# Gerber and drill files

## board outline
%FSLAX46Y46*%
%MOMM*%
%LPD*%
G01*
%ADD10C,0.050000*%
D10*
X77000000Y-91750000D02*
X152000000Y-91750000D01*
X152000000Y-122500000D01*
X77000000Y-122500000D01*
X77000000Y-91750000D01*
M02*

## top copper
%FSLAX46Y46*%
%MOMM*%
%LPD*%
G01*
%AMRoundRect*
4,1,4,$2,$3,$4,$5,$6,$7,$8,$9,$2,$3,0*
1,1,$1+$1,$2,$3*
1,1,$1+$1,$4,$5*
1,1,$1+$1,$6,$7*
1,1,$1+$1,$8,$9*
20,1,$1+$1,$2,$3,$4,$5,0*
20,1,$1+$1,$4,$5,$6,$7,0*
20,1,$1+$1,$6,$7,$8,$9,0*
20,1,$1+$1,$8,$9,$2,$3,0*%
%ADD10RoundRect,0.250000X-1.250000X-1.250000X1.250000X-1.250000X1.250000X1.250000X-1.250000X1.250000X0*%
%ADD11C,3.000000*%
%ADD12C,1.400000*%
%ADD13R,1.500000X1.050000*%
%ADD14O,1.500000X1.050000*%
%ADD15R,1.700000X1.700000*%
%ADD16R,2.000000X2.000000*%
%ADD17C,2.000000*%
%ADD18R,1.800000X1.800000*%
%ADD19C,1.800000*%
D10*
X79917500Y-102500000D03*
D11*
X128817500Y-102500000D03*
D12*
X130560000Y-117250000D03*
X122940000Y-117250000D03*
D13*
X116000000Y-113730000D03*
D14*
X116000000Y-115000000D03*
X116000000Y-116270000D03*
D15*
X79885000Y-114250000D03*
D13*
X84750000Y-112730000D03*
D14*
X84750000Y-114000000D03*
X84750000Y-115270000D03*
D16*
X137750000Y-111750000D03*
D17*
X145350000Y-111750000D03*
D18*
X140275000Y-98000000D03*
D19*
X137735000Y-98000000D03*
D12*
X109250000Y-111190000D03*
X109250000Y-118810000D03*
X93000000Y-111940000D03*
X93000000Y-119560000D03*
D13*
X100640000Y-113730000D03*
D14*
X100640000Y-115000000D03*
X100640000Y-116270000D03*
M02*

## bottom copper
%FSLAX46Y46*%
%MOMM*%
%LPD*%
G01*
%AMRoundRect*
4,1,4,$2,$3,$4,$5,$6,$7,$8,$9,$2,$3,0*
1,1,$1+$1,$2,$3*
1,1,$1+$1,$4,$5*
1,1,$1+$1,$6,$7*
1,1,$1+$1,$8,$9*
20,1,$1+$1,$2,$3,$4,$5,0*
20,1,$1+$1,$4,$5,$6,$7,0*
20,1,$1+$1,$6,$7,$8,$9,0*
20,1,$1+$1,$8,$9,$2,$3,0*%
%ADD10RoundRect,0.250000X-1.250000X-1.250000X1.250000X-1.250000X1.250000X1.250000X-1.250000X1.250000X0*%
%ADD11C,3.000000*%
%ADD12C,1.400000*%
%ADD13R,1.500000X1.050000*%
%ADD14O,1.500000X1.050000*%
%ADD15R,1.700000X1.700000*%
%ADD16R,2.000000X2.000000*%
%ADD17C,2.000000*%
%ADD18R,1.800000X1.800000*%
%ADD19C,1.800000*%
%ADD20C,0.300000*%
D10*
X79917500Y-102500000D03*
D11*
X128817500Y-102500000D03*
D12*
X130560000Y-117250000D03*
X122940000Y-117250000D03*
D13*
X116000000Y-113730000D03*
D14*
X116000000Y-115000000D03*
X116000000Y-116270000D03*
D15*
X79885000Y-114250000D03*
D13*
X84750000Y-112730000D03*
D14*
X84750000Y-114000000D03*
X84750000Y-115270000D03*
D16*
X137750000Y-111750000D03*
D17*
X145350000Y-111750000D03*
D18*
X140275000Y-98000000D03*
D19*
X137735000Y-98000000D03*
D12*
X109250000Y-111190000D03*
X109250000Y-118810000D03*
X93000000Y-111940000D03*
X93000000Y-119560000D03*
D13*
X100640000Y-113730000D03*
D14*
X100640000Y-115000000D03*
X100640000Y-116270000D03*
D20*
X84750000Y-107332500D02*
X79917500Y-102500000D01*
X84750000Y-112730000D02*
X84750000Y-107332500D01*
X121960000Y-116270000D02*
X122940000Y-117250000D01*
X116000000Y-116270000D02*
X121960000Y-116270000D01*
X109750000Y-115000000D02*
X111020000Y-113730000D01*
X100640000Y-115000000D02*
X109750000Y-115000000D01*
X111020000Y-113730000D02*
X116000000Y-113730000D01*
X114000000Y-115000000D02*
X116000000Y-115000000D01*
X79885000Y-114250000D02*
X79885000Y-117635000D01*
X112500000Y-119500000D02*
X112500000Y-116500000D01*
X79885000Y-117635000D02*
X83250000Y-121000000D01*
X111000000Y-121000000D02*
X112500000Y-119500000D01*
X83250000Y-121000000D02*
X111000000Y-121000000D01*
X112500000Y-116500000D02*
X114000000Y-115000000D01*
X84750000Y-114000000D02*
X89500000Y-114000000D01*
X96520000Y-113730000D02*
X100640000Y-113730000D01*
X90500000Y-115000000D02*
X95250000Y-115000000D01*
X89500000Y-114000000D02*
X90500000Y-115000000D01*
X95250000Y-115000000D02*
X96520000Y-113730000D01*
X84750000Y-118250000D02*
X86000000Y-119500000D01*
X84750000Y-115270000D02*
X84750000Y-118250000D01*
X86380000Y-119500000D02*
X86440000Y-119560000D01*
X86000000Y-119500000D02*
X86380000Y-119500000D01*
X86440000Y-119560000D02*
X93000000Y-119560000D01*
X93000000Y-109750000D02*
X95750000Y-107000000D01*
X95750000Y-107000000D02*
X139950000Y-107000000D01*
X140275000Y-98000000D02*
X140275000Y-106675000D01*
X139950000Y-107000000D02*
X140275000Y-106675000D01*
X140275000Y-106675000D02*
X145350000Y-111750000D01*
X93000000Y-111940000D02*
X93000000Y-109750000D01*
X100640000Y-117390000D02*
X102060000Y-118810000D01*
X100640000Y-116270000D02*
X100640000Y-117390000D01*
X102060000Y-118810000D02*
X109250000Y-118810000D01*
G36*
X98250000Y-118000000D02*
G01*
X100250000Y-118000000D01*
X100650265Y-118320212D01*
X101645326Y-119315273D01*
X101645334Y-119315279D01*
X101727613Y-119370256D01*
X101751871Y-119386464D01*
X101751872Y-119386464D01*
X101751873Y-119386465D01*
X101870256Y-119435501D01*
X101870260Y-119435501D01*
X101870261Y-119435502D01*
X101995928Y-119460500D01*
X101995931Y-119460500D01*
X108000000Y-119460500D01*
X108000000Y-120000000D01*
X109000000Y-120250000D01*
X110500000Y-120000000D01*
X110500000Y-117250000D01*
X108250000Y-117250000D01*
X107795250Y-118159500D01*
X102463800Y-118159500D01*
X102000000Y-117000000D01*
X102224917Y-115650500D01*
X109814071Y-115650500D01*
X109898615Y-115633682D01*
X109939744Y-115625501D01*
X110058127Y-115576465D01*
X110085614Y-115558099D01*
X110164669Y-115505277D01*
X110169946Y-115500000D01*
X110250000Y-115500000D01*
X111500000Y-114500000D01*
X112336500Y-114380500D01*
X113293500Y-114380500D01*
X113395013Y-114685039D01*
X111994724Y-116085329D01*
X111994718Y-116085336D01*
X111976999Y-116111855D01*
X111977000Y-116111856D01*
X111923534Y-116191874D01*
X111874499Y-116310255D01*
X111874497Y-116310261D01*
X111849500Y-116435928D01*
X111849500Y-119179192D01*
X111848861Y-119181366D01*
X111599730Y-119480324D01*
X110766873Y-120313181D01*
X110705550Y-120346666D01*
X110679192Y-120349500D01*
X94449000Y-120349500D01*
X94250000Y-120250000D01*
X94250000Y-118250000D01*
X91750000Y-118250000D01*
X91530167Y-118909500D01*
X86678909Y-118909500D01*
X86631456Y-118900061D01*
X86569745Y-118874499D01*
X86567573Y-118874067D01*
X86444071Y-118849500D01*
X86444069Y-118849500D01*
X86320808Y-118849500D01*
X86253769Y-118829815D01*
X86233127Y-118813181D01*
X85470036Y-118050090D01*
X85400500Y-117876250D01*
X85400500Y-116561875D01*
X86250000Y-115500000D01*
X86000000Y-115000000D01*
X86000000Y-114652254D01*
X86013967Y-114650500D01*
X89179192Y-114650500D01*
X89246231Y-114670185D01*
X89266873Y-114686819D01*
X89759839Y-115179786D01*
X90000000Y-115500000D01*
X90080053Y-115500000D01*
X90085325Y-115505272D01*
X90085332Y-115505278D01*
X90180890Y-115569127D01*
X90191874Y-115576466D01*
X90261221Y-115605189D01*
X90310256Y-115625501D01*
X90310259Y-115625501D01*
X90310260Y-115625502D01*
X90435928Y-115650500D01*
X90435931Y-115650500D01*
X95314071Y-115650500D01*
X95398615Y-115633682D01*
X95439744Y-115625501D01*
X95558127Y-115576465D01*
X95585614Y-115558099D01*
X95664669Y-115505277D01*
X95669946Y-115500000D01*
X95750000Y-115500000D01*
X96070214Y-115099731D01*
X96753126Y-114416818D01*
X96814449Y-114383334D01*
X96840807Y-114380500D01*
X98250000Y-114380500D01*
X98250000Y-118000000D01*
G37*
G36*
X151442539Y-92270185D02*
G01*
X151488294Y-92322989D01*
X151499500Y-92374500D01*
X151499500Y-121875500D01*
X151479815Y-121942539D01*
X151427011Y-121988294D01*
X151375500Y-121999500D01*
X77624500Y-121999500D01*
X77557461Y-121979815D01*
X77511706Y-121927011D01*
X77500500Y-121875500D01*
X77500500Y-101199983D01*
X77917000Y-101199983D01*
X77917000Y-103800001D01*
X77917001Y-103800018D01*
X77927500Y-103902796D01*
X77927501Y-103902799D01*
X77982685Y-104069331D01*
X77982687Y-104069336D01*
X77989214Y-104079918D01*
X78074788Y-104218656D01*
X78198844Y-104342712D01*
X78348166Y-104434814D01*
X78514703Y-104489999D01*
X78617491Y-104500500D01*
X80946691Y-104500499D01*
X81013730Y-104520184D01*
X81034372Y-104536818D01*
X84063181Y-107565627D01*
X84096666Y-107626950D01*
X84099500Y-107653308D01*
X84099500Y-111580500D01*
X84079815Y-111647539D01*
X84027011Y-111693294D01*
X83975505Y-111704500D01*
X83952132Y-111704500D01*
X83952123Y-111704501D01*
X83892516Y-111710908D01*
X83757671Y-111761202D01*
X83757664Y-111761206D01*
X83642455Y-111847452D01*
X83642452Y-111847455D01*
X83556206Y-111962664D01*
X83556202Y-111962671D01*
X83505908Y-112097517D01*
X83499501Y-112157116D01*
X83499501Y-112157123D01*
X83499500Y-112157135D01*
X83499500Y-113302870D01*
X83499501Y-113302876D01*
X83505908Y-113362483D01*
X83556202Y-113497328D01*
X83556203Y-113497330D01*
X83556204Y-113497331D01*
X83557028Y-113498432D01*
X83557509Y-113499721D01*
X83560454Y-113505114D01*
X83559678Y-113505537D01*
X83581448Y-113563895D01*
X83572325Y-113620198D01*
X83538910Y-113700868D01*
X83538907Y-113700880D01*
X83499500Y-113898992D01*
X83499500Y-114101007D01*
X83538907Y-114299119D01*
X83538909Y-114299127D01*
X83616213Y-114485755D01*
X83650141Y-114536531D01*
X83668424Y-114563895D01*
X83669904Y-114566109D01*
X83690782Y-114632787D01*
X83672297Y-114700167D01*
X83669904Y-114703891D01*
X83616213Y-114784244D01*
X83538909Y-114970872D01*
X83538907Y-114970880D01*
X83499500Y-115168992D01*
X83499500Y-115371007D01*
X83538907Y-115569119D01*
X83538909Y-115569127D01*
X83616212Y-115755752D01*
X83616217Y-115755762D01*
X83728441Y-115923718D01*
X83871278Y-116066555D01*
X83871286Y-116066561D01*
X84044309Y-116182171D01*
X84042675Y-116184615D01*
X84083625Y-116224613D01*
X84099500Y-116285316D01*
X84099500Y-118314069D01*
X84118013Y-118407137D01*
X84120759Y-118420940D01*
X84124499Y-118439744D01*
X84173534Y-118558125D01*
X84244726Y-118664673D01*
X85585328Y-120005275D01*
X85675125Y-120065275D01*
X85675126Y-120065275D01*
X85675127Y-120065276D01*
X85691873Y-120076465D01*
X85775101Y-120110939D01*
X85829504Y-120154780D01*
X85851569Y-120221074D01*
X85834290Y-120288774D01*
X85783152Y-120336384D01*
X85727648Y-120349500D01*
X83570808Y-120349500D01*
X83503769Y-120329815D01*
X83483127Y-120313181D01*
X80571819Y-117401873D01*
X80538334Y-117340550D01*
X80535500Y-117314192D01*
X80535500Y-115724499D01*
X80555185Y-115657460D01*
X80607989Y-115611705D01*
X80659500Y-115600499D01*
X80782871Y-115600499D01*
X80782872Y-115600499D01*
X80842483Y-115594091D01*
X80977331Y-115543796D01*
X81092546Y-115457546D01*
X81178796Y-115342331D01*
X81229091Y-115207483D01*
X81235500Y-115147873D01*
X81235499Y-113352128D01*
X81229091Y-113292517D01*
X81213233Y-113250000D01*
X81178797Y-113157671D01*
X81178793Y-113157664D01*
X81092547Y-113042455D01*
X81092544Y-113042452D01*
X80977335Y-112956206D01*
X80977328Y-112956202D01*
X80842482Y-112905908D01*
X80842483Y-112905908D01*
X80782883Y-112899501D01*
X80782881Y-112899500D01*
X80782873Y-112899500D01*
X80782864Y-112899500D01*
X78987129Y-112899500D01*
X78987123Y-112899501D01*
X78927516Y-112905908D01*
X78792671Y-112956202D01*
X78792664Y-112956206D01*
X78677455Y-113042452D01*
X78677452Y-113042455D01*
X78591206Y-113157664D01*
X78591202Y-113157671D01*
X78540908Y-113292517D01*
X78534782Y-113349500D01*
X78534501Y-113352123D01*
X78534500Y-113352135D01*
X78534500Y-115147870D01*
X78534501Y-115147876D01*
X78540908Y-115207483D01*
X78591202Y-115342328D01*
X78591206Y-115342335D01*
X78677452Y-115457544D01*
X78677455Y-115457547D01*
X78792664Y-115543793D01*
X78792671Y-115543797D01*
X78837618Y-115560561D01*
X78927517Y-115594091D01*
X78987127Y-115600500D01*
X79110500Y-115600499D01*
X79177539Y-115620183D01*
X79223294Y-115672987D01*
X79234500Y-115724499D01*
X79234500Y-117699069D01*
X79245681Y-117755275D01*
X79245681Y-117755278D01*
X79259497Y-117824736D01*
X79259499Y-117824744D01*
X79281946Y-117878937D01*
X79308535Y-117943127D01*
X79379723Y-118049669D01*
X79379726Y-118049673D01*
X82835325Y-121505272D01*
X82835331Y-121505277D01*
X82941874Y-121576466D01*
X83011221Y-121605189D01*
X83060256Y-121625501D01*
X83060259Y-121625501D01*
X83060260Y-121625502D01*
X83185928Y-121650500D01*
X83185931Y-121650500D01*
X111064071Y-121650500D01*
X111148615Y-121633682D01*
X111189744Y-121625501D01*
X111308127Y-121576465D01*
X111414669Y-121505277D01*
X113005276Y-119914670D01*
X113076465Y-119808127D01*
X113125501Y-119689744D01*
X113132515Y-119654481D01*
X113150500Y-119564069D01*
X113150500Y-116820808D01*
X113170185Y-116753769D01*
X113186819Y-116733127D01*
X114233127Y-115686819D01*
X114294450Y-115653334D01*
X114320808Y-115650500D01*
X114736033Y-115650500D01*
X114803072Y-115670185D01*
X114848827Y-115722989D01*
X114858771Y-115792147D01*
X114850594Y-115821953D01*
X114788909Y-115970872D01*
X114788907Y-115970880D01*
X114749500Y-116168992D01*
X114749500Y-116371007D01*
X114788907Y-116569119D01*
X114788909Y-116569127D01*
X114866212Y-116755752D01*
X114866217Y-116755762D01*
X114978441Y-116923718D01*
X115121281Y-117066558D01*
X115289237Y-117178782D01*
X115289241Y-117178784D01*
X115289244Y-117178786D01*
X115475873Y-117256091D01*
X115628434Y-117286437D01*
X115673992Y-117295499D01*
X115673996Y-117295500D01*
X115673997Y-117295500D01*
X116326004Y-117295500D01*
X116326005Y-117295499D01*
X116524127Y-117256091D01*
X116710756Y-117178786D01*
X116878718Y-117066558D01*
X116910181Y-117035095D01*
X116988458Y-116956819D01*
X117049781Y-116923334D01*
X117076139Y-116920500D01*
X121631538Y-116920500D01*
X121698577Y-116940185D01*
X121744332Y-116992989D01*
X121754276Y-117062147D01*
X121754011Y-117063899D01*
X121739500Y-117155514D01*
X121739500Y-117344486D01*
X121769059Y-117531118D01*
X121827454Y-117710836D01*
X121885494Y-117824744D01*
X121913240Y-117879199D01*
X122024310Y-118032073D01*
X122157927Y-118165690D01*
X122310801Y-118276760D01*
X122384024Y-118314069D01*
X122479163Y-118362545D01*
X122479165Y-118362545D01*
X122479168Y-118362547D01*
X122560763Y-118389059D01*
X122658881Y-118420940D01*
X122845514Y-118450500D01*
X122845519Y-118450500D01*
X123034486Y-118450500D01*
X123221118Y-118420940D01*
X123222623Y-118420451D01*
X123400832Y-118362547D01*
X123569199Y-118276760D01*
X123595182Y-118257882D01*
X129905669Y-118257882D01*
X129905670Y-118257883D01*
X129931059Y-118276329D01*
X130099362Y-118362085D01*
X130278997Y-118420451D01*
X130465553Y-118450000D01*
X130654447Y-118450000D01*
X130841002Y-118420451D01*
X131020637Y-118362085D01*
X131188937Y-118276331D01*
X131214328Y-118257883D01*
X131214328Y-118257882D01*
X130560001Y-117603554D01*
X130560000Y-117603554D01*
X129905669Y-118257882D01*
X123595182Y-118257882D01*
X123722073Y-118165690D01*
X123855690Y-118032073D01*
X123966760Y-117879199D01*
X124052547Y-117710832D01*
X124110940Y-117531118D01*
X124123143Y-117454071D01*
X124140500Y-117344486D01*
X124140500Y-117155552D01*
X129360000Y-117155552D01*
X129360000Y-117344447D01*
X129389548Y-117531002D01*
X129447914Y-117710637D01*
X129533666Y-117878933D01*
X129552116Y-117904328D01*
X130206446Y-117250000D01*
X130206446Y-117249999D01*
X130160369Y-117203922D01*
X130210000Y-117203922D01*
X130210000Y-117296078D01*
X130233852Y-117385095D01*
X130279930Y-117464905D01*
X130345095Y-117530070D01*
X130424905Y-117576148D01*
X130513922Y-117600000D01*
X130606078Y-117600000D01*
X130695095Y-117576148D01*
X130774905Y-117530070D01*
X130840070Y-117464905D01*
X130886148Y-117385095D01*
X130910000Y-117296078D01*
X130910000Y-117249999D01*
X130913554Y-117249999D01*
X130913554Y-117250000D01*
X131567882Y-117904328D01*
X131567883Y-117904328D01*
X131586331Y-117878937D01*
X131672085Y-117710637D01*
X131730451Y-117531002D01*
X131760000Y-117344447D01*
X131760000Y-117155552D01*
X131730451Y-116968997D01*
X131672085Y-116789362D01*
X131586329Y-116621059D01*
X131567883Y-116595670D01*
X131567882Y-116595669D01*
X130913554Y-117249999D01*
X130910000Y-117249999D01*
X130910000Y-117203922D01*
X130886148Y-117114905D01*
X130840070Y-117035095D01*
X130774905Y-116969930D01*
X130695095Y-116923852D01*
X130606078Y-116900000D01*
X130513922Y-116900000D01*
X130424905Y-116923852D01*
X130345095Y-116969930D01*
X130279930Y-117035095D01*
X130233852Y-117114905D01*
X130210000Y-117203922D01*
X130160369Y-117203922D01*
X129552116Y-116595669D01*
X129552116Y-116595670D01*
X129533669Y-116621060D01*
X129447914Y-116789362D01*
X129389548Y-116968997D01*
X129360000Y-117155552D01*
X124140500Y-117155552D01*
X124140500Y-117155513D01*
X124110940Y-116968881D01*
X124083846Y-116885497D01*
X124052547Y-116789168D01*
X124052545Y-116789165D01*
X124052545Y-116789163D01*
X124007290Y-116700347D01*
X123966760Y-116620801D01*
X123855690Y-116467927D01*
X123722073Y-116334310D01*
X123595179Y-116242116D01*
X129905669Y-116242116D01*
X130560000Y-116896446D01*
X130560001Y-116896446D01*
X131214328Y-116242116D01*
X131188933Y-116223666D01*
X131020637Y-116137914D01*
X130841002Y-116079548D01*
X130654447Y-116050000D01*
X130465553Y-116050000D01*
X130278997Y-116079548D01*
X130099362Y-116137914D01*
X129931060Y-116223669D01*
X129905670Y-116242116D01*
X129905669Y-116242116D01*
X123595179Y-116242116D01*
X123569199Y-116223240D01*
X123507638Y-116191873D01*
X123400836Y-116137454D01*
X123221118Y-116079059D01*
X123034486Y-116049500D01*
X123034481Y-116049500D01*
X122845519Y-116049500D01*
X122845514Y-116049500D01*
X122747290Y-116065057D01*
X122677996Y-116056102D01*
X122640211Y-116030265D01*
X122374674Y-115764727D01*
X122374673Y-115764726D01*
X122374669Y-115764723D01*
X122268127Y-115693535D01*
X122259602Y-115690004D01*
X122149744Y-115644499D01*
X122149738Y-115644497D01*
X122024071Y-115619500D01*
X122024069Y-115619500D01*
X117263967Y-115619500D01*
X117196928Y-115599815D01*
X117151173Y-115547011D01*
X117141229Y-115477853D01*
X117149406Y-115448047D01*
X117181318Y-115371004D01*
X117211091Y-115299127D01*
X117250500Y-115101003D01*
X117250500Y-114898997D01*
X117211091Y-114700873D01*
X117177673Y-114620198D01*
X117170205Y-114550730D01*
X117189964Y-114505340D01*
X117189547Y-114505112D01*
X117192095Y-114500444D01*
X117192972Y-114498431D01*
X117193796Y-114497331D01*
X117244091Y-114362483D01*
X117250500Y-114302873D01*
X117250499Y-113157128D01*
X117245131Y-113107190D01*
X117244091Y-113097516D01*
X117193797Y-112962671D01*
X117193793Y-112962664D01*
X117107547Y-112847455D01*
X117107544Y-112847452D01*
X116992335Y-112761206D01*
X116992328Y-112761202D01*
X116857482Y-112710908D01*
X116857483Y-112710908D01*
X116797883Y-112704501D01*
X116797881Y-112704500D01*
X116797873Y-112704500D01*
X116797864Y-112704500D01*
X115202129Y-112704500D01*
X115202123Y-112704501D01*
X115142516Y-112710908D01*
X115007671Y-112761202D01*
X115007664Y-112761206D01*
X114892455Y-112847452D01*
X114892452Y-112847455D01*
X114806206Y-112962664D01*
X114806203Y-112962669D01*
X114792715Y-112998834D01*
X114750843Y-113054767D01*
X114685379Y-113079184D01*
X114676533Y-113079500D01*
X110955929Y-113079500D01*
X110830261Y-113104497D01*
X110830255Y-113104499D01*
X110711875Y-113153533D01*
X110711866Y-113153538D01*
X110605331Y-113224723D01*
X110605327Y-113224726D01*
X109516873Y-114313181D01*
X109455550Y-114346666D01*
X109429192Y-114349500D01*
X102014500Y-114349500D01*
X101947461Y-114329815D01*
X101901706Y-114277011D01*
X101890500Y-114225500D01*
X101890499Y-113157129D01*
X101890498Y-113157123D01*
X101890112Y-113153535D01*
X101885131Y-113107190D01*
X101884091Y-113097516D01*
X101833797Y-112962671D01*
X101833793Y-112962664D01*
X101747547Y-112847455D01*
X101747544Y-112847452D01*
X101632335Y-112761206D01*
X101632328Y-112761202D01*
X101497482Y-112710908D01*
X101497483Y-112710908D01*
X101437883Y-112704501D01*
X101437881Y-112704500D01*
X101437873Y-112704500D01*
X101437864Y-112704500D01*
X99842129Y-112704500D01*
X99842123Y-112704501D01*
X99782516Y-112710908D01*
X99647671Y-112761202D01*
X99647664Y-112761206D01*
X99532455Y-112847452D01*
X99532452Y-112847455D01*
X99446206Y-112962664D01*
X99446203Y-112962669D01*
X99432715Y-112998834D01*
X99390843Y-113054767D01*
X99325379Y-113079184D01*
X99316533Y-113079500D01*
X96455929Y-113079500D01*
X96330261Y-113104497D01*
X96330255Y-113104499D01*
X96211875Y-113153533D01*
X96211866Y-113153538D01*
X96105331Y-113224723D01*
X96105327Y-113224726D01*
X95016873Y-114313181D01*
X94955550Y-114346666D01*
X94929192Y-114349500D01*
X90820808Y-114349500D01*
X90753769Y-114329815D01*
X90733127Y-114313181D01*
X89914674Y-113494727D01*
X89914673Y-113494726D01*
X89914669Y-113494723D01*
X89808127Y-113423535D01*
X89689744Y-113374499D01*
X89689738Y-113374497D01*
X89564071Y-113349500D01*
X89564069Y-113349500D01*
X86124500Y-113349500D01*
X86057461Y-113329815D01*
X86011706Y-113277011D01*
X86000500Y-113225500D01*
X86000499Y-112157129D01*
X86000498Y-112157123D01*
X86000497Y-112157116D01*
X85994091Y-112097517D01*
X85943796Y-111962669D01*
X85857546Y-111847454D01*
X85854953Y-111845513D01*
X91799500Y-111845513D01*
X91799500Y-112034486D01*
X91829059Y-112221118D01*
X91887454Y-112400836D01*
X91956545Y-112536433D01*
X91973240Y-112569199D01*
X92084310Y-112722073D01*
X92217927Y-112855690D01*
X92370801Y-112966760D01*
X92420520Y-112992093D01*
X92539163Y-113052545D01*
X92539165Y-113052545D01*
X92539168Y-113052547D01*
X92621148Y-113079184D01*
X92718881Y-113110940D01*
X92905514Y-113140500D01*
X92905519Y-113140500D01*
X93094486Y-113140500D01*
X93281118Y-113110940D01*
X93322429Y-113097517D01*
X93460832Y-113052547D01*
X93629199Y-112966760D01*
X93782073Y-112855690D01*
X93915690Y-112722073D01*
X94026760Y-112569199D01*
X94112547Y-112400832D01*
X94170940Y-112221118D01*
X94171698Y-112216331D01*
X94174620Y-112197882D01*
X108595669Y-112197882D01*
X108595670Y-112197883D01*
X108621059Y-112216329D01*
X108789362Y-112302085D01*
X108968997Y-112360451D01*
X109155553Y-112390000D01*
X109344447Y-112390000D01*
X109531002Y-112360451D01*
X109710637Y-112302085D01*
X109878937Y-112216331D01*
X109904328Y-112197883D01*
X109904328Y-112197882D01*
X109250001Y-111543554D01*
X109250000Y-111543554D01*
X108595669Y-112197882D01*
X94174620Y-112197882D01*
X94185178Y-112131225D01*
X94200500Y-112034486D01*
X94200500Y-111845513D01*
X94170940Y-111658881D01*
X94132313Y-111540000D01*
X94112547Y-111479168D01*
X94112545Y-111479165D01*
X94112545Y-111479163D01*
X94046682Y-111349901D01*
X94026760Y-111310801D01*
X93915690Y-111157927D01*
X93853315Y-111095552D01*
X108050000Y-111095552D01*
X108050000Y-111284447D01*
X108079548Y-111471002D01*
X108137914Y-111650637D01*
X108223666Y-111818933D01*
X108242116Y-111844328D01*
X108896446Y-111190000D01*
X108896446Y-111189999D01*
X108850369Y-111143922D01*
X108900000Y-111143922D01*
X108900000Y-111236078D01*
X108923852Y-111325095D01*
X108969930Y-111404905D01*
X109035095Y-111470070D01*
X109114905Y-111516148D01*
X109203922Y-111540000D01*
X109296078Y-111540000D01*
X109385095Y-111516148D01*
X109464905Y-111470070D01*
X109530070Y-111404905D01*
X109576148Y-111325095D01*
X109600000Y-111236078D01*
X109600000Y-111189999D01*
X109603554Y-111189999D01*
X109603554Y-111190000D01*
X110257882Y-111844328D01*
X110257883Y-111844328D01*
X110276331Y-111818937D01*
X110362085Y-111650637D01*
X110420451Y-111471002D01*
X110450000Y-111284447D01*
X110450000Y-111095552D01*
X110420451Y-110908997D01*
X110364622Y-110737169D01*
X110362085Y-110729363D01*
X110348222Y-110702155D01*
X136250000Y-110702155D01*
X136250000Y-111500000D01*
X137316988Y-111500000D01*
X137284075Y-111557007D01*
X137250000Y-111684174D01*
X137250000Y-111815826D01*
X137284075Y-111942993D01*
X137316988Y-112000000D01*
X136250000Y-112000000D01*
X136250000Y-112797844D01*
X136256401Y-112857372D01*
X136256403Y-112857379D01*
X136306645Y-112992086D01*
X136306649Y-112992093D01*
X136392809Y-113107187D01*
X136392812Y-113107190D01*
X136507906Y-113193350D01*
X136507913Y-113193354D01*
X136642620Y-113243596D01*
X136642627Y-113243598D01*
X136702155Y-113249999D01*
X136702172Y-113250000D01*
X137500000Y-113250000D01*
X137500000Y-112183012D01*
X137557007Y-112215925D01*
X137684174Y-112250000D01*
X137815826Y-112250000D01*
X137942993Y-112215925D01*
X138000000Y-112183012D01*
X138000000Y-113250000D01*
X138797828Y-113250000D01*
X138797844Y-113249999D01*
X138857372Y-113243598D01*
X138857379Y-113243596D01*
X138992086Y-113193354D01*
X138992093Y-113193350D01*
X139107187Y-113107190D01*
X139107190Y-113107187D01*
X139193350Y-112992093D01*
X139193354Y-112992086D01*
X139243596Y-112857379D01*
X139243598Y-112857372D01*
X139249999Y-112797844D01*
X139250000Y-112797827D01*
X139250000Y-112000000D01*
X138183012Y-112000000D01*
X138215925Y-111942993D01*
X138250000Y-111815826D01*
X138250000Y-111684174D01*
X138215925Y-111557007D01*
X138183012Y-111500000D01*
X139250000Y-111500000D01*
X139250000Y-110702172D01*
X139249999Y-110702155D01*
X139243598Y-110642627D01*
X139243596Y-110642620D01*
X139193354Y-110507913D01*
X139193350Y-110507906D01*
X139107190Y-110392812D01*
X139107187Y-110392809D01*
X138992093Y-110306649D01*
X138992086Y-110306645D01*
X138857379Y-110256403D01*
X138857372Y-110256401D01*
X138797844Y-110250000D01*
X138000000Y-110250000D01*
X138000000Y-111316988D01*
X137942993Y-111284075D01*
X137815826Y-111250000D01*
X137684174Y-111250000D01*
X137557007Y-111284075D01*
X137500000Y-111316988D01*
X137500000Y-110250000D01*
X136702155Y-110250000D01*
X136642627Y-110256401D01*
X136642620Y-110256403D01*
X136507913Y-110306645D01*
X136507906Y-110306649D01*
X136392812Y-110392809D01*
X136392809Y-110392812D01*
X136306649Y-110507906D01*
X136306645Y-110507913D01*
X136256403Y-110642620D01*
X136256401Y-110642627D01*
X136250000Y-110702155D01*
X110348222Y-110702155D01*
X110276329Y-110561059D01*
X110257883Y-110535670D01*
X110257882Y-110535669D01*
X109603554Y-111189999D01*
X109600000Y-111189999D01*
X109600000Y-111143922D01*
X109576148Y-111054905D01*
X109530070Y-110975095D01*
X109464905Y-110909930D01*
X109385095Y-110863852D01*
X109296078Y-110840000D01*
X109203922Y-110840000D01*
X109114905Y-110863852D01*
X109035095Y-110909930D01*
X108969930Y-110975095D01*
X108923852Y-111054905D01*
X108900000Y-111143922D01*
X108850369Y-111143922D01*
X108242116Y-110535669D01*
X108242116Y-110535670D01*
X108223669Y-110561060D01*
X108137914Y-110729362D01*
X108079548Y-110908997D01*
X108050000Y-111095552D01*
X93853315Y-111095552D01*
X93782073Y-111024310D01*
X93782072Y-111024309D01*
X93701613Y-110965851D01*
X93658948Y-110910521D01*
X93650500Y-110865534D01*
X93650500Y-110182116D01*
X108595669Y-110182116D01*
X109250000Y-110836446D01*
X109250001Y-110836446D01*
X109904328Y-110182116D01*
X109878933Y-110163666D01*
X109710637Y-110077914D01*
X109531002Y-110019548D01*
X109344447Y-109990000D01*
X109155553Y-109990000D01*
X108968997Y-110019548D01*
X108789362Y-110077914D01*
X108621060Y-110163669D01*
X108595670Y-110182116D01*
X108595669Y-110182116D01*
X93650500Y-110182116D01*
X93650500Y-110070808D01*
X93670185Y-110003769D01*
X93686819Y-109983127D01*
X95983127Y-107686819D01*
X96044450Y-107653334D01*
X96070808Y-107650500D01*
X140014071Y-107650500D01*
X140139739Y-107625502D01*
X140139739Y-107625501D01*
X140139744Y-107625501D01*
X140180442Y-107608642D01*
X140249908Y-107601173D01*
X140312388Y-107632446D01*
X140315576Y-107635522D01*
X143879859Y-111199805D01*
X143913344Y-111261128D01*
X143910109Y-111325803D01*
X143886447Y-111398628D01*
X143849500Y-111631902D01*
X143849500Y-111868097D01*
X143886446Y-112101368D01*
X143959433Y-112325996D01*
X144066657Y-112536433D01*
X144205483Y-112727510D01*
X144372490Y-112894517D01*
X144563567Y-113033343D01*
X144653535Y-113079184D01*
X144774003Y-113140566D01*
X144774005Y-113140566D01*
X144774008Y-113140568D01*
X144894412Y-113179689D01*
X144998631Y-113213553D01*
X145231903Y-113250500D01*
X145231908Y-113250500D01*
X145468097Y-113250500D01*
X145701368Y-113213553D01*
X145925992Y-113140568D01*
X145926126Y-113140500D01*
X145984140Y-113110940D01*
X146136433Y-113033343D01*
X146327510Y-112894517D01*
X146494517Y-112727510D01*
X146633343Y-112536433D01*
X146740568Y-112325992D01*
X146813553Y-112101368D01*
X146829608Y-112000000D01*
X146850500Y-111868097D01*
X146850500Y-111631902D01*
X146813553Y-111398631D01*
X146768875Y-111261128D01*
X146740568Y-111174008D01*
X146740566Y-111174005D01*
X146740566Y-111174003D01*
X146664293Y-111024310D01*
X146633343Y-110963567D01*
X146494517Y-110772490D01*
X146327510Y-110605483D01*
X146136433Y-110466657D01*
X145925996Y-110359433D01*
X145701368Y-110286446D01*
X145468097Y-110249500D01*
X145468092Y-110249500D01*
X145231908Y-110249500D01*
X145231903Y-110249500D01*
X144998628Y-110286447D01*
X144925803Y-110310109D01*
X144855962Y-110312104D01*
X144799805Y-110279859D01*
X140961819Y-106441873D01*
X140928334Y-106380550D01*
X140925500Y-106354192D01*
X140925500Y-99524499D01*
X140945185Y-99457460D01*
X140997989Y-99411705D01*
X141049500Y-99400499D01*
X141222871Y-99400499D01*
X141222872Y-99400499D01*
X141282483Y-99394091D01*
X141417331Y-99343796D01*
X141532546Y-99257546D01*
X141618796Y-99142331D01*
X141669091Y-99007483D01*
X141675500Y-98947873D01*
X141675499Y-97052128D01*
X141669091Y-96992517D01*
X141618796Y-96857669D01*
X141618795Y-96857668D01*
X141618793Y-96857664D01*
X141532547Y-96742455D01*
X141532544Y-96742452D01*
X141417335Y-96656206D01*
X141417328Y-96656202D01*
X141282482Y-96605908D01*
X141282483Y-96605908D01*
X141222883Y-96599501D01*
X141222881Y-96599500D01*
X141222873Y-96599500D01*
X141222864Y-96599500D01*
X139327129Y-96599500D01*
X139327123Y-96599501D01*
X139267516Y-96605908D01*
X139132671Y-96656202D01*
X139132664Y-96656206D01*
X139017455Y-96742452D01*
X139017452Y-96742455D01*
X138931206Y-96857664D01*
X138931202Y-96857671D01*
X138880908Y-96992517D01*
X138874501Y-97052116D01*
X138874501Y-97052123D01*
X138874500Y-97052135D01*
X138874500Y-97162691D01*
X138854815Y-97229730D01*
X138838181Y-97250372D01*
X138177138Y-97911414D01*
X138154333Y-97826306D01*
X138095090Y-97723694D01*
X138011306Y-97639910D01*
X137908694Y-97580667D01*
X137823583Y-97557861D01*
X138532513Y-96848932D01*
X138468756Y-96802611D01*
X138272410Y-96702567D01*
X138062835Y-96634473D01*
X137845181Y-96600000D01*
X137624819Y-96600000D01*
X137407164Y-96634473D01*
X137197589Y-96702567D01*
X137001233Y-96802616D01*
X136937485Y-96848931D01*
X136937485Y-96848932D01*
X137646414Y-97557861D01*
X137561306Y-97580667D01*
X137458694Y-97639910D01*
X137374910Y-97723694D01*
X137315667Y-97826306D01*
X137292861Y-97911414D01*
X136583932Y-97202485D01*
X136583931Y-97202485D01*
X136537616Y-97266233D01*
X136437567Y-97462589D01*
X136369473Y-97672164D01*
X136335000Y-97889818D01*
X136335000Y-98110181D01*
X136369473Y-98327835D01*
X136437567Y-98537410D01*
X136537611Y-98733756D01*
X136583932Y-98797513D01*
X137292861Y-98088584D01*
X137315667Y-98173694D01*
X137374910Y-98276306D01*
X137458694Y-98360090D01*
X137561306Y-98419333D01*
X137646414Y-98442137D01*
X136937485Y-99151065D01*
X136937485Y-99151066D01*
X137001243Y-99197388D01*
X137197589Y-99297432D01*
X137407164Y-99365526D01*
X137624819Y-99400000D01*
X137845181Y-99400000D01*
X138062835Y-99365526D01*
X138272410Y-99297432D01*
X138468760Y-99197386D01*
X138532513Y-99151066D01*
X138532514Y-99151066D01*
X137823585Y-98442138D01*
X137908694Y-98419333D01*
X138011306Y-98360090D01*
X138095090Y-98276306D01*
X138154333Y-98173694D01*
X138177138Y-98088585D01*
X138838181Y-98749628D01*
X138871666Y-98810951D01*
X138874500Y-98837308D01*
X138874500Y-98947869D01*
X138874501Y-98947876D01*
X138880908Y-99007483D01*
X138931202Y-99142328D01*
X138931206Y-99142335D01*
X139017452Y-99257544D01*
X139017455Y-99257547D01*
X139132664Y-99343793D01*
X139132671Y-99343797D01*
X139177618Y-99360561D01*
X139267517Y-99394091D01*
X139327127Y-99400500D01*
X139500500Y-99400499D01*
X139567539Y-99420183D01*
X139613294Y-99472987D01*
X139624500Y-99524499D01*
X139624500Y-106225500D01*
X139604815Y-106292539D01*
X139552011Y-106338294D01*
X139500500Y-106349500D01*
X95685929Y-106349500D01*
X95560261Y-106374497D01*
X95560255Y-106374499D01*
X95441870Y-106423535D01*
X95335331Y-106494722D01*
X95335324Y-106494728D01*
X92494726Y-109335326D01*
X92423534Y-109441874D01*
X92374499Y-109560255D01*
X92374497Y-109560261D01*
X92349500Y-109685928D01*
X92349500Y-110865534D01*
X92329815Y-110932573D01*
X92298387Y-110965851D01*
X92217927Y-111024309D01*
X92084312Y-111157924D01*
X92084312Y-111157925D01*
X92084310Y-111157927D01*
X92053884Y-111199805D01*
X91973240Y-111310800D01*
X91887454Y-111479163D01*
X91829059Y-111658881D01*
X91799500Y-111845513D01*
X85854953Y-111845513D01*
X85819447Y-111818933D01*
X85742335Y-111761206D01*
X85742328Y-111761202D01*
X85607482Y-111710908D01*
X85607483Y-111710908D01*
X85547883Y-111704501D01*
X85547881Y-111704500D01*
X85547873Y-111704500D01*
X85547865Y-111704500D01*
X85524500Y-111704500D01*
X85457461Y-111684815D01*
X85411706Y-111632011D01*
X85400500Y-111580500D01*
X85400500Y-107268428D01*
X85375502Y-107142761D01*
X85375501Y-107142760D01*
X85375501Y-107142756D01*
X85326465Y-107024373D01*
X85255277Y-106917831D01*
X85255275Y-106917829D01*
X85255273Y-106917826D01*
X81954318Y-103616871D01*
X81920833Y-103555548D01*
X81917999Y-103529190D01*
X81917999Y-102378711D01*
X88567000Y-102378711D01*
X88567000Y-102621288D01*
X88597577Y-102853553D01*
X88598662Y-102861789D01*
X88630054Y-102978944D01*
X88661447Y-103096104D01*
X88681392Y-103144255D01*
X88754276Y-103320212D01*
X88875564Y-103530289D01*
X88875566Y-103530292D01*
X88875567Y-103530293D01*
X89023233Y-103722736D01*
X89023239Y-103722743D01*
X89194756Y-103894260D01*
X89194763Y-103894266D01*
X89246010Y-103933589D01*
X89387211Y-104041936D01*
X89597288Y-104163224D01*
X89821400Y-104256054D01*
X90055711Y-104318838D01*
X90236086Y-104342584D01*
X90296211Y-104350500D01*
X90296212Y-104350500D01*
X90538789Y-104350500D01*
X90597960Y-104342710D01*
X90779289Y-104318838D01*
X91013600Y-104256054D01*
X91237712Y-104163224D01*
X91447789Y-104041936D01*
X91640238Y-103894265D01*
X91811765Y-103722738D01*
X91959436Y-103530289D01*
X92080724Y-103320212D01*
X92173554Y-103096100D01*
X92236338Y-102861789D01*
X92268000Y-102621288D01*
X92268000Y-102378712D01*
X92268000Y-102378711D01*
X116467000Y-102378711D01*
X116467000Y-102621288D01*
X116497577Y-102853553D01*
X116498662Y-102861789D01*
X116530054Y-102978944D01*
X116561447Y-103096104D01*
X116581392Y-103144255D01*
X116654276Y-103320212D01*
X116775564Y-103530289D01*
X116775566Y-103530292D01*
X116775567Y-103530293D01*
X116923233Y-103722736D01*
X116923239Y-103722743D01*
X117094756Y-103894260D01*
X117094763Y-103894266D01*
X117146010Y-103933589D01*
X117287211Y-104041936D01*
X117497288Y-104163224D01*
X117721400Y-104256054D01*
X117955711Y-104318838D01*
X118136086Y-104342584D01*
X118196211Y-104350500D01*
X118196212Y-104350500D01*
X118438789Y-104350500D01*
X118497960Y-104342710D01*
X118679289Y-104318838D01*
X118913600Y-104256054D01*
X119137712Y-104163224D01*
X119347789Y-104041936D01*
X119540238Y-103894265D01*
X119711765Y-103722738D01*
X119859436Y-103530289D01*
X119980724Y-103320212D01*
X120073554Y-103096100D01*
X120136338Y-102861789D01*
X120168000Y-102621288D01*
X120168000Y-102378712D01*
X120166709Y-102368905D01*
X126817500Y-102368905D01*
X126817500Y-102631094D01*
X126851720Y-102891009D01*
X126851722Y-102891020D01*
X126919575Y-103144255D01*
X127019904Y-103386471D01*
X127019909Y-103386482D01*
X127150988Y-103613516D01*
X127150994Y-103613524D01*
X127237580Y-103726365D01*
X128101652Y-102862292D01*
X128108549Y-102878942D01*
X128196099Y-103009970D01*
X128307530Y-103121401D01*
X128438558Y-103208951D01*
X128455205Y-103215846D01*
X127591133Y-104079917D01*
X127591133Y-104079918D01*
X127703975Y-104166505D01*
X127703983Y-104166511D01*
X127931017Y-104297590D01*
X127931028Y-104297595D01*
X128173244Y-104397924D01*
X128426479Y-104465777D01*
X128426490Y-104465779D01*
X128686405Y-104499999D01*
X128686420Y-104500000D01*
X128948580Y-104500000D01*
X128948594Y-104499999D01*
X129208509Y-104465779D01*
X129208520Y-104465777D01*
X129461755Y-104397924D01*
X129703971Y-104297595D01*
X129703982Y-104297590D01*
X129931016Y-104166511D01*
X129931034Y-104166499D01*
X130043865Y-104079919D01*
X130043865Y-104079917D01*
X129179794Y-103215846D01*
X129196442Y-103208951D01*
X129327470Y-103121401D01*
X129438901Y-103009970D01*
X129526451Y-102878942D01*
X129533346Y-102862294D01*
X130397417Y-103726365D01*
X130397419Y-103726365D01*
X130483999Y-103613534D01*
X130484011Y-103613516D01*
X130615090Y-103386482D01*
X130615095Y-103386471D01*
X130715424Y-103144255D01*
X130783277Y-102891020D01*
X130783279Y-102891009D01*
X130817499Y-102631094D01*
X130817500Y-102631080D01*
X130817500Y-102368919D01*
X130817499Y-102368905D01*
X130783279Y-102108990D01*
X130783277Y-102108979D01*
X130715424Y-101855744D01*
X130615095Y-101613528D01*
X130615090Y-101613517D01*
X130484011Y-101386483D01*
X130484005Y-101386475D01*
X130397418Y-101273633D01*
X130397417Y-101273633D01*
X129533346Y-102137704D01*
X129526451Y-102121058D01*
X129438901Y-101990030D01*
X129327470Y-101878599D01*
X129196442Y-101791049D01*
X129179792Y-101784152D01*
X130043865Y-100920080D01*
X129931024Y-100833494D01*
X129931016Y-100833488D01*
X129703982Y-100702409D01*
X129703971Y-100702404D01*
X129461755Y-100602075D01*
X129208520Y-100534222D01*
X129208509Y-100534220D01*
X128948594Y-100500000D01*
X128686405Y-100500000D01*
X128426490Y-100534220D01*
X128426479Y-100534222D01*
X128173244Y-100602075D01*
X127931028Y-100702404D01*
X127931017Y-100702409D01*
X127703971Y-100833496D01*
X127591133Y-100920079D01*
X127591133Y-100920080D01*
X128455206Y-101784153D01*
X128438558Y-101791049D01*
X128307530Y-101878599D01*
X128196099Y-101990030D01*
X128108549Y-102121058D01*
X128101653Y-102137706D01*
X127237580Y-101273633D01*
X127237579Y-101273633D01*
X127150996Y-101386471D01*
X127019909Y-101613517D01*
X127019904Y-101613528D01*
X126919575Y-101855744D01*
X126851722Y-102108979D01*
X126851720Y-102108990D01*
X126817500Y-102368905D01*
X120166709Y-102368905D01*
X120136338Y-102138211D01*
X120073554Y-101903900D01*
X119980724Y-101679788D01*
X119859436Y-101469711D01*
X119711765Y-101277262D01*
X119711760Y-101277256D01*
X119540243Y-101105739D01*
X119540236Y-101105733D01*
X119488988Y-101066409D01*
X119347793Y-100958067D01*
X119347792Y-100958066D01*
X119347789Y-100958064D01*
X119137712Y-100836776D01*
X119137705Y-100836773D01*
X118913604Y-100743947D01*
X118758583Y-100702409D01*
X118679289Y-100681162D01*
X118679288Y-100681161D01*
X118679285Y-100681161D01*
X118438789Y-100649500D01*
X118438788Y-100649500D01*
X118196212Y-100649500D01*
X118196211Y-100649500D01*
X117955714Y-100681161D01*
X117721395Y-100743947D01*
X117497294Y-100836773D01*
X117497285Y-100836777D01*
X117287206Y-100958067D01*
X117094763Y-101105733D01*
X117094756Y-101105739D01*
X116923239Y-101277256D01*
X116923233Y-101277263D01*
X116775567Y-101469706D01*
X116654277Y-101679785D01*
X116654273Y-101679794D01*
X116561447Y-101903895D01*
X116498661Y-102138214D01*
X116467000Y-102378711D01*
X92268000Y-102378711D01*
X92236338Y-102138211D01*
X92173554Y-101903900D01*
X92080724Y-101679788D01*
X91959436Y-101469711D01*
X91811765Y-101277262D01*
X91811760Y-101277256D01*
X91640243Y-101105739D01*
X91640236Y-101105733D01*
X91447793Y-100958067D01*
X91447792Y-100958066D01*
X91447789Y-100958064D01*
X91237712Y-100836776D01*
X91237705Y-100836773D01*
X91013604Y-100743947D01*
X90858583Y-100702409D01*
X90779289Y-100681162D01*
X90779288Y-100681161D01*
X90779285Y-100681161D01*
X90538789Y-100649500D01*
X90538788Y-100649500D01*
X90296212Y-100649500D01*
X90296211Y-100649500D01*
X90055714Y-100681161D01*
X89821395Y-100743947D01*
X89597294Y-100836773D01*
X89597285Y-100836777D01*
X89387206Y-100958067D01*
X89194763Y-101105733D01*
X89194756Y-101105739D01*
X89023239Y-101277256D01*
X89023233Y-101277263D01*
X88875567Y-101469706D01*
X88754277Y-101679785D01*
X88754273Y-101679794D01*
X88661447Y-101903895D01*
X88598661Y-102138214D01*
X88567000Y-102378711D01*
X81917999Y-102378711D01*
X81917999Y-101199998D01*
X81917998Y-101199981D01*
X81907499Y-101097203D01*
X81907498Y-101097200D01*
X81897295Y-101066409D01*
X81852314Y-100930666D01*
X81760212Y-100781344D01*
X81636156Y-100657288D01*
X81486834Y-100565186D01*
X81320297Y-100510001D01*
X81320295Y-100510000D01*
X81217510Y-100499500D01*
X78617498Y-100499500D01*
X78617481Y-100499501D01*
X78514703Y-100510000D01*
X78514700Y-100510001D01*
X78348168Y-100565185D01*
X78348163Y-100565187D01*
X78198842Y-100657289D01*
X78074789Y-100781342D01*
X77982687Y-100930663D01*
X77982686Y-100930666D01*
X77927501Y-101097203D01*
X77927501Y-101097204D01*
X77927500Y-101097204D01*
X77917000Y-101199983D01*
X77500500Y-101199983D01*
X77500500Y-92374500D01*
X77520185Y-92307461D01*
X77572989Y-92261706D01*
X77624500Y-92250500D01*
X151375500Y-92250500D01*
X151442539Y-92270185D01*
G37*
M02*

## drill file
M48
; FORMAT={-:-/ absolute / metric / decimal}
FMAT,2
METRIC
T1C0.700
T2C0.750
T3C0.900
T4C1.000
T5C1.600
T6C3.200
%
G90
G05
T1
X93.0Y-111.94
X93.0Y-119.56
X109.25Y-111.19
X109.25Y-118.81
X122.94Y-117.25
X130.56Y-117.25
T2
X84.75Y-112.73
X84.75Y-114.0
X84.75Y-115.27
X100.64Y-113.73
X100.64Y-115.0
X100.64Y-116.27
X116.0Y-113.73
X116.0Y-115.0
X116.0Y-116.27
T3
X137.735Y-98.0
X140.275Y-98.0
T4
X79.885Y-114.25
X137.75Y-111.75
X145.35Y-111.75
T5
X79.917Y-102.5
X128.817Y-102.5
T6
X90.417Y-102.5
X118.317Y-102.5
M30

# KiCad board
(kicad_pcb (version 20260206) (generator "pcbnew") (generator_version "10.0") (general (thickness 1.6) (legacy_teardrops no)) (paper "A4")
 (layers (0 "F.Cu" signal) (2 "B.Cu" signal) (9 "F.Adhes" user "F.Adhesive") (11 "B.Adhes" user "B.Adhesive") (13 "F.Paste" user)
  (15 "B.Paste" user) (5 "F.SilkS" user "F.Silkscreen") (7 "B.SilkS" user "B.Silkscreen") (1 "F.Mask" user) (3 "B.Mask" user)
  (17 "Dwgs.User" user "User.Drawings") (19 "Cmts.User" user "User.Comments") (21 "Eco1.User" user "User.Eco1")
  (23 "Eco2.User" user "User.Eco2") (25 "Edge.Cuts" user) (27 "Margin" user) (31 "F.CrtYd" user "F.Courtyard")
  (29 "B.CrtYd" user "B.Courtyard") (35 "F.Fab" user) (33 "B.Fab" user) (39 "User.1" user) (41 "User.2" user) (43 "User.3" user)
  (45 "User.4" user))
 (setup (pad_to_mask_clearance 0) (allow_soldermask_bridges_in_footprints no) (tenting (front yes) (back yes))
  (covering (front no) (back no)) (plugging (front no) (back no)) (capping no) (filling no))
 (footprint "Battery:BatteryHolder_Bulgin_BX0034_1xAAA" (layer "F.Cu") (at 79.9175 102.5)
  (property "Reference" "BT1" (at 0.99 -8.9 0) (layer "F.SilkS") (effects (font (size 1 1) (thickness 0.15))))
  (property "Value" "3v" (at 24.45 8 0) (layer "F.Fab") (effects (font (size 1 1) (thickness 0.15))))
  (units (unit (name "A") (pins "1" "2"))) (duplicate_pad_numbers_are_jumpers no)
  (pad "" np_thru_hole circle (at 10.5 0) (size 3.2 3.2) (drill 3.2) (layers "*.Cu" "*.Mask"))
  (pad "" np_thru_hole circle (at 38.4 0) (size 3.2 3.2) (drill 3.2) (layers "*.Cu" "*.Mask"))
  (pad "1" thru_hole roundrect (at 0 0) (size 3 3) (drill 1.6) (layers "*.Cu" "*.Mask") (remove_unused_layers no)
   (roundrect_rratio 0.08333333333) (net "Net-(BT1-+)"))
  (pad "2" thru_hole circle (at 48.9 0) (size 3 3) (drill 1.6) (layers "*.Cu" "*.Mask") (remove_unused_layers no) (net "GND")))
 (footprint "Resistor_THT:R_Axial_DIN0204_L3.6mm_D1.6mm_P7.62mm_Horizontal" (layer "F.Cu") (at 130.56 117.25 180)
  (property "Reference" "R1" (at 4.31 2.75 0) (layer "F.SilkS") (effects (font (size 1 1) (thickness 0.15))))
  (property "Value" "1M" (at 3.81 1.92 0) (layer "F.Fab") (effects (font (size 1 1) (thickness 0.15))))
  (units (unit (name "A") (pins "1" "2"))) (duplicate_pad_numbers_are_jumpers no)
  (pad "1" thru_hole circle (at 0 0 180) (size 1.4 1.4) (drill 0.7) (layers "*.Cu" "*.Mask") (remove_unused_layers no) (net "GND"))
  (pad "2" thru_hole circle (at 7.62 0 180) (size 1.4 1.4) (drill 0.7) (layers "*.Cu" "*.Mask") (remove_unused_layers no) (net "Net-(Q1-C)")))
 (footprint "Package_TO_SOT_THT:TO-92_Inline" (layer "F.Cu") (at 116 113.73 -90)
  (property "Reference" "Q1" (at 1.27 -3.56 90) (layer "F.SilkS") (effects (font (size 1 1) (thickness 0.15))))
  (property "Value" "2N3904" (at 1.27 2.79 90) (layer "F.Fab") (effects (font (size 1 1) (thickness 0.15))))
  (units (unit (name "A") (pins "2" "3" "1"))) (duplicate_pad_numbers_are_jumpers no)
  (pad "1" thru_hole rect (at 0 0 270) (size 1.05 1.5) (drill 0.75) (layers "*.Cu" "*.Mask") (remove_unused_layers no) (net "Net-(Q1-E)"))
  (pad "2" thru_hole oval (at 1.27 0 270) (size 1.05 1.5) (drill 0.75) (layers "*.Cu" "*.Mask") (remove_unused_layers no)
   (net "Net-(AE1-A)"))
  (pad "3" thru_hole oval (at 2.54 0 270) (size 1.05 1.5) (drill 0.75) (layers "*.Cu" "*.Mask") (remove_unused_layers no) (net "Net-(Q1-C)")))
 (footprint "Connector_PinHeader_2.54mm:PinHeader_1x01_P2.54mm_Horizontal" (layer "F.Cu") (at 79.885 114.25 180)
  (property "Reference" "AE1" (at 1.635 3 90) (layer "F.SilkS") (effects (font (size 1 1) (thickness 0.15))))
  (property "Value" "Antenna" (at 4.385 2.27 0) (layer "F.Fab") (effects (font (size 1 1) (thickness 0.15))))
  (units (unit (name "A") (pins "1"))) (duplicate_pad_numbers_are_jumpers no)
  (pad "1" thru_hole rect (at 0 0 180) (size 1.7 1.7) (drill 1) (layers "*.Cu" "*.Mask") (remove_unused_layers no) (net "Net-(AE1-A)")))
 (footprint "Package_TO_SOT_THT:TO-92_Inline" (layer "F.Cu") (at 84.75 112.73 -90)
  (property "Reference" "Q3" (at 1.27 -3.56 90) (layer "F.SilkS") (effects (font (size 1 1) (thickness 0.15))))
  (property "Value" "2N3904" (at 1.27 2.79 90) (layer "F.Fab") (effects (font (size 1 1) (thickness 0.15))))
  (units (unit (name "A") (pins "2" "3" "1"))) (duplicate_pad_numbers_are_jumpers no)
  (pad "1" thru_hole rect (at 0 0 270) (size 1.05 1.5) (drill 0.75) (layers "*.Cu" "*.Mask") (remove_unused_layers no) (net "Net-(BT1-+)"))
  (pad "2" thru_hole oval (at 1.27 0 270) (size 1.05 1.5) (drill 0.75) (layers "*.Cu" "*.Mask") (remove_unused_layers no) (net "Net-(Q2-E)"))
  (pad "3" thru_hole oval (at 2.54 0 270) (size 1.05 1.5) (drill 0.75) (layers "*.Cu" "*.Mask") (remove_unused_layers no) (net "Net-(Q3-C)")))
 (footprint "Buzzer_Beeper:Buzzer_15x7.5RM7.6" (layer "F.Cu") (at 137.75 111.75)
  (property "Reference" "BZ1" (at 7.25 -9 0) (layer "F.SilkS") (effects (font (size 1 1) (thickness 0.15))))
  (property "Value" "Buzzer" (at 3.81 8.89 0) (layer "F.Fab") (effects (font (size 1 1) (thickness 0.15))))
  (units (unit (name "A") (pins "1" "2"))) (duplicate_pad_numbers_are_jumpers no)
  (pad "1" thru_hole rect (at 0 0) (size 2 2) (drill 1) (layers "*.Cu" "*.Mask") (remove_unused_layers no) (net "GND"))
  (pad "2" thru_hole circle (at 7.6 0) (size 2 2) (drill 1) (layers "*.Cu" "*.Mask") (remove_unused_layers no) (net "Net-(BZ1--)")))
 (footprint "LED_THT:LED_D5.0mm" (layer "F.Cu") (at 140.275 98 180)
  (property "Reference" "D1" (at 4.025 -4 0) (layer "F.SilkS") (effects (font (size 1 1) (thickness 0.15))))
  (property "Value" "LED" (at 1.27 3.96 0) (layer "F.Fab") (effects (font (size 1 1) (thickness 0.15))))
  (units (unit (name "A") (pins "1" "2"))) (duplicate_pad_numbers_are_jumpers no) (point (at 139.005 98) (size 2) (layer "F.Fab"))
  (pad "1" thru_hole rect (at 0 0 180) (size 1.8 1.8) (drill 0.9) (layers "*.Cu" "*.Mask") (remove_unused_layers no) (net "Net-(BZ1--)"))
  (pad "2" thru_hole circle (at 2.54 0 180) (size 1.8 1.8) (drill 0.9) (layers "*.Cu" "*.Mask") (remove_unused_layers no) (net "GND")))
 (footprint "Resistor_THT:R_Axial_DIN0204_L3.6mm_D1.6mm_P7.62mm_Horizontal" (layer "F.Cu") (at 109.25 111.19 -90)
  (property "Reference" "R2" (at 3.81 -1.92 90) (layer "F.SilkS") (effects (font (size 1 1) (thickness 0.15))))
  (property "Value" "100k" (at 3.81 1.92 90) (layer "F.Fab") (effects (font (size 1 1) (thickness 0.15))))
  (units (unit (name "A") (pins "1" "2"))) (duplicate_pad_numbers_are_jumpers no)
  (pad "1" thru_hole circle (at 0 0 270) (size 1.4 1.4) (drill 0.7) (layers "*.Cu" "*.Mask") (remove_unused_layers no) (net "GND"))
  (pad "2" thru_hole circle (at 7.62 0 270) (size 1.4 1.4) (drill 0.7) (layers "*.Cu" "*.Mask") (remove_unused_layers no) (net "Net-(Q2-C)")))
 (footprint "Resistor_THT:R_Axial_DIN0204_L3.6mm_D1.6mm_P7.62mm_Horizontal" (layer "F.Cu") (at 93 111.94 -90)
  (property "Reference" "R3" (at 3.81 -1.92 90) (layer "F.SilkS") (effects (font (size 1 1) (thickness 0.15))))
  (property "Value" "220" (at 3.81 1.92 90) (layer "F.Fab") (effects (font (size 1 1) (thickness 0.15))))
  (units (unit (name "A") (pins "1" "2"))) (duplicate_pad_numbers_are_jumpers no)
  (pad "1" thru_hole circle (at 0 0 270) (size 1.4 1.4) (drill 0.7) (layers "*.Cu" "*.Mask") (remove_unused_layers no) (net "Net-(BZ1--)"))
  (pad "2" thru_hole circle (at 7.62 0 270) (size 1.4 1.4) (drill 0.7) (layers "*.Cu" "*.Mask") (remove_unused_layers no) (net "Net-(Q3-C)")))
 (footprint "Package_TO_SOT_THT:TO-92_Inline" (layer "F.Cu") (at 100.64 113.73 -90)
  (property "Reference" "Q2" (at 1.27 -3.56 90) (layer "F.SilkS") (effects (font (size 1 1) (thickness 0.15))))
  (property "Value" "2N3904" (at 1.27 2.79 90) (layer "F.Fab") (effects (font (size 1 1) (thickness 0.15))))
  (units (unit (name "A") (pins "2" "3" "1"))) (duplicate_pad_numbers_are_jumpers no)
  (pad "1" thru_hole rect (at 0 0 270) (size 1.05 1.5) (drill 0.75) (layers "*.Cu" "*.Mask") (remove_unused_layers no) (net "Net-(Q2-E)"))
  (pad "2" thru_hole oval (at 1.27 0 270) (size 1.05 1.5) (drill 0.75) (layers "*.Cu" "*.Mask") (remove_unused_layers no) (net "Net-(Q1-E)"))
  (pad "3" thru_hole oval (at 2.54 0 270) (size 1.05 1.5) (drill 0.75) (layers "*.Cu" "*.Mask") (remove_unused_layers no) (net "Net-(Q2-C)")))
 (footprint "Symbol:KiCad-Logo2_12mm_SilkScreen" (layer "B.Cu") (at 107.764893 102.267106)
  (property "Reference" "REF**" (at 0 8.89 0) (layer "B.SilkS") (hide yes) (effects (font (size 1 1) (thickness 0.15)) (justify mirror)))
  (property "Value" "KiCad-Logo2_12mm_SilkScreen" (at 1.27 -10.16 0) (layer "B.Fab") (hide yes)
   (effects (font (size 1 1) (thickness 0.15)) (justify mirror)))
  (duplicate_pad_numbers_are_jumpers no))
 (gr_rect (start 77 91.75) (end 152 122.5) (stroke (width 0.05) (type default)) (fill no) (layer "Edge.Cuts"))
 (segment (start 84.75 107.3325) (end 79.9175 102.5) (width 0.3) (layer "B.Cu") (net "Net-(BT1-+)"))
 (segment (start 84.75 112.73) (end 84.75 107.3325) (width 0.3) (layer "B.Cu") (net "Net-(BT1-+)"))
 (segment (start 121.96 116.27) (end 122.94 117.25) (width 0.3) (layer "B.Cu") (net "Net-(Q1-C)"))
 (segment (start 116 116.27) (end 121.96 116.27) (width 0.3) (layer "B.Cu") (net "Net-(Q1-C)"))
 (segment (start 109.75 115) (end 111.02 113.73) (width 0.3) (layer "B.Cu") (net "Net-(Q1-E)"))
 (segment (start 100.64 115) (end 109.75 115) (width 0.3) (layer "B.Cu") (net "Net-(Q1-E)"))
 (segment (start 111.02 113.73) (end 116 113.73) (width 0.3) (layer "B.Cu") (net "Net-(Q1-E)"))
 (segment (start 114 115) (end 116 115) (width 0.3) (layer "B.Cu") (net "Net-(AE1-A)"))
 (segment (start 79.885 114.25) (end 79.885 117.635) (width 0.3) (layer "B.Cu") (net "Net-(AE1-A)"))
 (segment (start 112.5 119.5) (end 112.5 116.5) (width 0.3) (layer "B.Cu") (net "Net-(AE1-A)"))
 (segment (start 79.885 117.635) (end 83.25 121) (width 0.3) (layer "B.Cu") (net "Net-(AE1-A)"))
 (segment (start 111 121) (end 112.5 119.5) (width 0.3) (layer "B.Cu") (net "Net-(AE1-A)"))
 (segment (start 83.25 121) (end 111 121) (width 0.3) (layer "B.Cu") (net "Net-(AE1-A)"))
 (segment (start 112.5 116.5) (end 114 115) (width 0.3) (layer "B.Cu") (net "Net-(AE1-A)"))
 (segment (start 84.75 114) (end 89.5 114) (width 0.3) (layer "B.Cu") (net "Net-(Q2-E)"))
 (segment (start 96.52 113.73) (end 100.64 113.73) (width 0.3) (layer "B.Cu") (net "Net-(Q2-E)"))
 (segment (start 90.5 115) (end 95.25 115) (width 0.3) (layer "B.Cu") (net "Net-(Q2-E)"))
 (segment (start 89.5 114) (end 90.5 115) (width 0.3) (layer "B.Cu") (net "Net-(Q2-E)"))
 (segment (start 95.25 115) (end 96.52 113.73) (width 0.3) (layer "B.Cu") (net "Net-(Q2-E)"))
 (segment (start 84.75 118.25) (end 86 119.5) (width 0.3) (layer "B.Cu") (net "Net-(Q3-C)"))
 (segment (start 84.75 115.27) (end 84.75 118.25) (width 0.3) (layer "B.Cu") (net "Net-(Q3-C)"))
 (segment (start 86.38 119.5) (end 86.44 119.56) (width 0.3) (layer "B.Cu") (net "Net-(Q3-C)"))
 (segment (start 86 119.5) (end 86.38 119.5) (width 0.3) (layer "B.Cu") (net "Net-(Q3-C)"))
 (segment (start 86.44 119.56) (end 93 119.56) (width 0.3) (layer "B.Cu") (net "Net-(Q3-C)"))
 (segment (start 93 109.75) (end 95.75 107) (width 0.3) (layer "B.Cu") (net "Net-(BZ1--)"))
 (segment (start 95.75 107) (end 139.95 107) (width 0.3) (layer "B.Cu") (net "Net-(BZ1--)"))
 (segment (start 140.275 98) (end 140.275 106.675) (width 0.3) (layer "B.Cu") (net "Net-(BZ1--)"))
 (segment (start 139.95 107) (end 140.275 106.675) (width 0.3) (layer "B.Cu") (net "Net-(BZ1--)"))
 (segment (start 140.275 106.675) (end 145.35 111.75) (width 0.3) (layer "B.Cu") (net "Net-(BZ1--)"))
 (segment (start 93 111.94) (end 93 109.75) (width 0.3) (layer "B.Cu") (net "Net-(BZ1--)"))
 (segment (start 100.64 117.39) (end 102.06 118.81) (width 0.3) (layer "B.Cu") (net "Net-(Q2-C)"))
 (segment (start 100.64 116.27) (end 100.64 117.39) (width 0.3) (layer "B.Cu") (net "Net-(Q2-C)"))
 (segment (start 102.06 118.81) (end 109.25 118.81) (width 0.3) (layer "B.Cu") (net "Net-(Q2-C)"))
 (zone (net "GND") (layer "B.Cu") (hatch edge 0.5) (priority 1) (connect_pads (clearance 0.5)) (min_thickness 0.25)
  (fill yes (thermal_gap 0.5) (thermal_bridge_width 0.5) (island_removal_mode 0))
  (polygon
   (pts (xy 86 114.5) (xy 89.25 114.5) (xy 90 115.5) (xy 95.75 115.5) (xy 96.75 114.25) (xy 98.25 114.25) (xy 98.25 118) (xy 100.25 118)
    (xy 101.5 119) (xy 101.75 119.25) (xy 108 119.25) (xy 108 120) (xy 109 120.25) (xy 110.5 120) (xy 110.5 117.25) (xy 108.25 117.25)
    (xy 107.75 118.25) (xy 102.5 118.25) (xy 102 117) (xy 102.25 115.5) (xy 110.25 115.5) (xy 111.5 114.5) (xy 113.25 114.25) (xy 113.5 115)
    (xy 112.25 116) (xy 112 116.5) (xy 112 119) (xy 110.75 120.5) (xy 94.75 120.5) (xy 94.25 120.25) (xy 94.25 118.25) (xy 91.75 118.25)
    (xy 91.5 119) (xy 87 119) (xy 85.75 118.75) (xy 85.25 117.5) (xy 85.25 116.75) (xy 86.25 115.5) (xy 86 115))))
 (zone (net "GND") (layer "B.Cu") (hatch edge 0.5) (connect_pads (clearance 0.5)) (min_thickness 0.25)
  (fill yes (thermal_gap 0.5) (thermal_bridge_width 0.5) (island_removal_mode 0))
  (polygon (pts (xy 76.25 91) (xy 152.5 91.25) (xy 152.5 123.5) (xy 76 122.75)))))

